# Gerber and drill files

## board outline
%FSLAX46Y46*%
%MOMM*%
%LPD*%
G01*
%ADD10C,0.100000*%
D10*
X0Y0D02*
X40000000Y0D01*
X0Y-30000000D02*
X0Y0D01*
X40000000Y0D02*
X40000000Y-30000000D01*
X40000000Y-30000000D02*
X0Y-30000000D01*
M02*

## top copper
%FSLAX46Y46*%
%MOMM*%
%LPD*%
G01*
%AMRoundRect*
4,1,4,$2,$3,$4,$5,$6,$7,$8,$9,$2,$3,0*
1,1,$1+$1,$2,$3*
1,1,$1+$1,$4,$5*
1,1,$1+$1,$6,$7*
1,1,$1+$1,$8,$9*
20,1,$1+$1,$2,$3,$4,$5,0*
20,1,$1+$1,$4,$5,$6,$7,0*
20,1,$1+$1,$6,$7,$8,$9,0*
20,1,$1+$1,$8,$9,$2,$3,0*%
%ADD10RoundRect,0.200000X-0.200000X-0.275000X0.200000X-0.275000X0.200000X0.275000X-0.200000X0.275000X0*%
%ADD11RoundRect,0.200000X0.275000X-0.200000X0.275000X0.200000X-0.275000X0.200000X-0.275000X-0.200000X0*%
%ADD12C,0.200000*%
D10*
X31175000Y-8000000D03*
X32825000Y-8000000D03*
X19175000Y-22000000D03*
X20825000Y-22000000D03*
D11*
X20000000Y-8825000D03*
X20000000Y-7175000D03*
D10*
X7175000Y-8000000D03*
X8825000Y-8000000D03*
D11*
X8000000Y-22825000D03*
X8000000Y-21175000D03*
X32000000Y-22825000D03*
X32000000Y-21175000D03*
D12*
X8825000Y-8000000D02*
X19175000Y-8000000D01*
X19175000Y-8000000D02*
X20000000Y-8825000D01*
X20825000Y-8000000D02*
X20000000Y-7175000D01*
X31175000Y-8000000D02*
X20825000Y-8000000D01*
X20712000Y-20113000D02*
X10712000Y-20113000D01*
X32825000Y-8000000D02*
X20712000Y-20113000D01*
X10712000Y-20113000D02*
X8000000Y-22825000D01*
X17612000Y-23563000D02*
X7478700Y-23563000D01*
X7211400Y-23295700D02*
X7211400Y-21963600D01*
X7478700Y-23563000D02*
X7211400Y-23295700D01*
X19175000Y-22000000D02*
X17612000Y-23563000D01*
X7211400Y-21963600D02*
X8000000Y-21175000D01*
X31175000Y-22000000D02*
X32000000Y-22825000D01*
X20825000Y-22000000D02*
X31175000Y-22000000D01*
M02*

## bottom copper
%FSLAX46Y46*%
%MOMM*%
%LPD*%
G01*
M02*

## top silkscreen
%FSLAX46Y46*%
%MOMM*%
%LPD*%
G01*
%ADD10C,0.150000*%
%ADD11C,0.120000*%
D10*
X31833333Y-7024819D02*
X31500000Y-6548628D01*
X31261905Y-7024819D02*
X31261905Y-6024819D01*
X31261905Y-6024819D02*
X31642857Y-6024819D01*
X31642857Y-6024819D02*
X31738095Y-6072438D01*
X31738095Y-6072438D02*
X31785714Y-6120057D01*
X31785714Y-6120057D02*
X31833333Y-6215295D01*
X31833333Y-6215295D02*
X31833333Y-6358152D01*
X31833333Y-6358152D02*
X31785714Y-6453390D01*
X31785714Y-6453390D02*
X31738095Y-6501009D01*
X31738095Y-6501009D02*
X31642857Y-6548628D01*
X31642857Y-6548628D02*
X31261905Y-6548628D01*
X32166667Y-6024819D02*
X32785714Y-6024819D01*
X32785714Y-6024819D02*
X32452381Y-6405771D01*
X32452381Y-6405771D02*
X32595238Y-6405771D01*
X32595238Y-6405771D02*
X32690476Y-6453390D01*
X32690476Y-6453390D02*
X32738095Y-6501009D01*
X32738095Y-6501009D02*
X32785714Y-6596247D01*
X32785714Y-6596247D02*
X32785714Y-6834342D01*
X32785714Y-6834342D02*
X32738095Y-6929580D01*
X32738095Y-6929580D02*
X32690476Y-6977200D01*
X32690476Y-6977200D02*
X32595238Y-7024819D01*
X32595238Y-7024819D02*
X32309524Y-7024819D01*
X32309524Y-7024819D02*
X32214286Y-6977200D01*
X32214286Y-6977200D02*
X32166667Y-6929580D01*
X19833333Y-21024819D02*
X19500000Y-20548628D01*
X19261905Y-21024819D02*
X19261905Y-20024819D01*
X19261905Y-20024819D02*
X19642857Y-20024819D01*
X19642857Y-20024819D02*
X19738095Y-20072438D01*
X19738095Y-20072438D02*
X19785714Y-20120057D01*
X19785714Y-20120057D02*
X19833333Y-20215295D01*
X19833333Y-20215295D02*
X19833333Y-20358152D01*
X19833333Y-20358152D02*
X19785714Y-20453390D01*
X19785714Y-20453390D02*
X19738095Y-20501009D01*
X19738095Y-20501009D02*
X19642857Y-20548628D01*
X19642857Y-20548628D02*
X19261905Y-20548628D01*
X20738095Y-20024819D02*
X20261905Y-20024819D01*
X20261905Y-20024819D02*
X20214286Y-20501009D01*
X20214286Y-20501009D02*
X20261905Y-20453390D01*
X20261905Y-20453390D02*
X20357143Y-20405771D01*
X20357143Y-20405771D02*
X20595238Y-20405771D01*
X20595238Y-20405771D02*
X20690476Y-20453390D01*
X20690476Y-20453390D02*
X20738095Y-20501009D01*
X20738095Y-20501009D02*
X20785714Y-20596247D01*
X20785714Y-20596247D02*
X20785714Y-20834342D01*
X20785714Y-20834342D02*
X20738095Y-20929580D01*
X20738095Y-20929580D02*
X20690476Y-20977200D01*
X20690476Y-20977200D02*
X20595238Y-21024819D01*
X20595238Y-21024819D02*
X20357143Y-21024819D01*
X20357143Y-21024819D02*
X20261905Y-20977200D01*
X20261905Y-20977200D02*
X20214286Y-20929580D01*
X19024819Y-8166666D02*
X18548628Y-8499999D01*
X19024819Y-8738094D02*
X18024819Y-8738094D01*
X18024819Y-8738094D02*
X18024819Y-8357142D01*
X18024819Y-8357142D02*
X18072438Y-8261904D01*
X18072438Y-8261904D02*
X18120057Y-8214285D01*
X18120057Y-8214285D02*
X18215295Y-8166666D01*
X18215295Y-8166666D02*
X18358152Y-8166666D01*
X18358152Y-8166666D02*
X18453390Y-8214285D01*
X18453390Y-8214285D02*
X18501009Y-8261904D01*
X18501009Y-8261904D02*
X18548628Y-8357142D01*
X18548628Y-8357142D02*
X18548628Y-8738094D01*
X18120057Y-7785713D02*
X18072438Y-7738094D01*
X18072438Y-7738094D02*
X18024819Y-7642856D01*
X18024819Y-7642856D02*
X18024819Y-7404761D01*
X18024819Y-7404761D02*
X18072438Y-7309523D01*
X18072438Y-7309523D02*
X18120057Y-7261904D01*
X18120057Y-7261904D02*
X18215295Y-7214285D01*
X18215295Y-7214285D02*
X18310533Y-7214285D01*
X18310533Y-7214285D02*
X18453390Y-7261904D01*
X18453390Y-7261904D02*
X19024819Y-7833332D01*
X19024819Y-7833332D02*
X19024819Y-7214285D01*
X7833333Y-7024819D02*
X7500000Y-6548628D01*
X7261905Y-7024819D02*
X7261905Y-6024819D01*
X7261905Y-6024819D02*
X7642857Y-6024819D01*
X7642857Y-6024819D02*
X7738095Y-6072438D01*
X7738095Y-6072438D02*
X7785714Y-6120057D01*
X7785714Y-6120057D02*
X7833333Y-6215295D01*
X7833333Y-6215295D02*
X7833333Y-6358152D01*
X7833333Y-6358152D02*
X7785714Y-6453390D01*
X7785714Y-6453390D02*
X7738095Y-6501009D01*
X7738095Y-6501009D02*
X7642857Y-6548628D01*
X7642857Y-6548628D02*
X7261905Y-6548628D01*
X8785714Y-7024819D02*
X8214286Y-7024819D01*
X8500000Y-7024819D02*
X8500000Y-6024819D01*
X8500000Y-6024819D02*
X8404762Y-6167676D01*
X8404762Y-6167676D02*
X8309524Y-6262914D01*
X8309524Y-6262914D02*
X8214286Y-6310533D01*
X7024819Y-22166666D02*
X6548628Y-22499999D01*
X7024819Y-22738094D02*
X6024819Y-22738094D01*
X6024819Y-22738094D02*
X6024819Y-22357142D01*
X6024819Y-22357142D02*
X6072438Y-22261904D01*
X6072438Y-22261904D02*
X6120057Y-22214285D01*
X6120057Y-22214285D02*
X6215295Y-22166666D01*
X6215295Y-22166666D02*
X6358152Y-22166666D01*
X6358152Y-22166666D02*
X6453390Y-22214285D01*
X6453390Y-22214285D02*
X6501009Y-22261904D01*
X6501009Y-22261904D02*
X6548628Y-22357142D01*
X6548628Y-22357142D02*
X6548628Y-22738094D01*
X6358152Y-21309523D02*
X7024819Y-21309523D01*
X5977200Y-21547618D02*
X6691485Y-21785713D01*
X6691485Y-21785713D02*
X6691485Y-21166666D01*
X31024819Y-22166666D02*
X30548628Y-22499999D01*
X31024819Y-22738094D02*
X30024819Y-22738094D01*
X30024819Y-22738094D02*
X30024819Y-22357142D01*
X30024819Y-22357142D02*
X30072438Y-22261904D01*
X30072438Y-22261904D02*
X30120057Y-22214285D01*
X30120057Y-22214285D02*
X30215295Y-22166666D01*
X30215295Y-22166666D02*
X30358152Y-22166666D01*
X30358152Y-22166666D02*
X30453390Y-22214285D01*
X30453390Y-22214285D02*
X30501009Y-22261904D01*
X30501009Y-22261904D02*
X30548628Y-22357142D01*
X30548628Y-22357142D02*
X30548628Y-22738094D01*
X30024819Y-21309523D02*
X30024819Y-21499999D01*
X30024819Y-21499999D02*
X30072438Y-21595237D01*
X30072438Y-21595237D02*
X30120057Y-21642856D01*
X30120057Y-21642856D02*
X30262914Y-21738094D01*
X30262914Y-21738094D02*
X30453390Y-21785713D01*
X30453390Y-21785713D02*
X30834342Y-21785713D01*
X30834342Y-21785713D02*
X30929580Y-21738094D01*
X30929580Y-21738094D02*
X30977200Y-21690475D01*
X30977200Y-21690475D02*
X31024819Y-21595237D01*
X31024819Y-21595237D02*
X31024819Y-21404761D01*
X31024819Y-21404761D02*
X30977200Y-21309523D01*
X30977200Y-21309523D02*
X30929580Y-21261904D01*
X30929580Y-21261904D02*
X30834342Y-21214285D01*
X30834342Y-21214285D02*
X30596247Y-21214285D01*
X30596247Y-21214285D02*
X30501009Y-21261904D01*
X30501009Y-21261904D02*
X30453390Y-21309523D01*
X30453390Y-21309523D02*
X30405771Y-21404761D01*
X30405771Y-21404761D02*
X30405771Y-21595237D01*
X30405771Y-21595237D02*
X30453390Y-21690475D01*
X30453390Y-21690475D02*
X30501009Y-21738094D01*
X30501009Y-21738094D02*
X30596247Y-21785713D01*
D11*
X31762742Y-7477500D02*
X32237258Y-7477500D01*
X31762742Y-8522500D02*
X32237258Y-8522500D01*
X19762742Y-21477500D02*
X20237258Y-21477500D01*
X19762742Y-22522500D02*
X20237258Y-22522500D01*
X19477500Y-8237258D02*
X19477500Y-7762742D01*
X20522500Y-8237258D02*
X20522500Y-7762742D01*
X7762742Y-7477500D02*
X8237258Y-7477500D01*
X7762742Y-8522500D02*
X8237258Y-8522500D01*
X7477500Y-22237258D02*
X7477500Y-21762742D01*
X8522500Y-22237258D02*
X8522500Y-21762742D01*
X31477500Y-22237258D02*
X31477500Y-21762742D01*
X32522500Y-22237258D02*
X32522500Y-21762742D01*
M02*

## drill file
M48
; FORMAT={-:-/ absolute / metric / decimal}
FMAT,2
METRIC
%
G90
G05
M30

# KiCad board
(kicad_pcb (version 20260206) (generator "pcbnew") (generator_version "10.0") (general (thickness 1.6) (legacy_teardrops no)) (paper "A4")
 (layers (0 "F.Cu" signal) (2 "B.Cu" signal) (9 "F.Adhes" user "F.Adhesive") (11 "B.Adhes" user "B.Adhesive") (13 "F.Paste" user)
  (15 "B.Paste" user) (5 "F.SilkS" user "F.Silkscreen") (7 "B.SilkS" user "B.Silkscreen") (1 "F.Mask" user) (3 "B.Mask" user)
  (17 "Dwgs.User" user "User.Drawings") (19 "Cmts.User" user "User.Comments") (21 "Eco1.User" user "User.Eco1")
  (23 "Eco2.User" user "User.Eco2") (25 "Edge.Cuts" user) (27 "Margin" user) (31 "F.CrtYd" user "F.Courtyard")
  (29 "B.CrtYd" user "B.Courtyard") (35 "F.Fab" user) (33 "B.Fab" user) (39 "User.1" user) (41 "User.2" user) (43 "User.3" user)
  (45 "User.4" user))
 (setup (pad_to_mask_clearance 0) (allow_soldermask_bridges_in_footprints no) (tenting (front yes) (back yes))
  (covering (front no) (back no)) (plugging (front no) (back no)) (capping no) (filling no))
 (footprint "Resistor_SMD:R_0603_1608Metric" (layer "F.Cu") (at 32 8)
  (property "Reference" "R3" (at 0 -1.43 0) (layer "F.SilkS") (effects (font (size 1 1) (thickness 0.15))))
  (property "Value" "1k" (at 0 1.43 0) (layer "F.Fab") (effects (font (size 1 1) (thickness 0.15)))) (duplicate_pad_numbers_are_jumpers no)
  (fp_line (start -0.237258 -0.5225) (end 0.237258 -0.5225) (stroke (width 0.12) (type solid)) (layer "F.SilkS"))
  (fp_line (start -0.237258 0.5225) (end 0.237258 0.5225) (stroke (width 0.12) (type solid)) (layer "F.SilkS"))
  (pad "1" smd roundrect (at -0.825 0) (size 0.8 0.95) (layers "F.Cu" "F.Mask" "F.Paste") (roundrect_rratio 0.25) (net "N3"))
  (pad "2" smd roundrect (at 0.825 0) (size 0.8 0.95) (layers "F.Cu" "F.Mask" "F.Paste") (roundrect_rratio 0.25) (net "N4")))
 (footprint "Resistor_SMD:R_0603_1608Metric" (layer "F.Cu") (at 20 22)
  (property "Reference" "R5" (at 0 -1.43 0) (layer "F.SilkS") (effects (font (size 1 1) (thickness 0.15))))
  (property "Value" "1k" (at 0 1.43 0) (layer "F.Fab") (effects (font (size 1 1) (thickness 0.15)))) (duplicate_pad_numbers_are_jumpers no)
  (fp_line (start -0.237258 -0.5225) (end 0.237258 -0.5225) (stroke (width 0.12) (type solid)) (layer "F.SilkS"))
  (fp_line (start -0.237258 0.5225) (end 0.237258 0.5225) (stroke (width 0.12) (type solid)) (layer "F.SilkS"))
  (pad "1" smd roundrect (at -0.825 0) (size 0.8 0.95) (layers "F.Cu" "F.Mask" "F.Paste") (roundrect_rratio 0.25) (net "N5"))
  (pad "2" smd roundrect (at 0.825 0) (size 0.8 0.95) (layers "F.Cu" "F.Mask" "F.Paste") (roundrect_rratio 0.25) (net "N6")))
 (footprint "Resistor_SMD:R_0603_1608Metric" (layer "F.Cu") (at 20 8 90)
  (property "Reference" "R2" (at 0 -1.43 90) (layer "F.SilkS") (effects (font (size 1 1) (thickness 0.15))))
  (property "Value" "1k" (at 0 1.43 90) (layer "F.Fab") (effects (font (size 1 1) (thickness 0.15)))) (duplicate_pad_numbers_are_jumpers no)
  (fp_line (start -0.237258 -0.5225) (end 0.237258 -0.5225) (stroke (width 0.12) (type solid)) (layer "F.SilkS"))
  (fp_line (start -0.237258 0.5225) (end 0.237258 0.5225) (stroke (width 0.12) (type solid)) (layer "F.SilkS"))
  (pad "1" smd roundrect (at -0.825 0 90) (size 0.8 0.95) (layers "F.Cu" "F.Mask" "F.Paste") (roundrect_rratio 0.25) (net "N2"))
  (pad "2" smd roundrect (at 0.825 0 90) (size 0.8 0.95) (layers "F.Cu" "F.Mask" "F.Paste") (roundrect_rratio 0.25) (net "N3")))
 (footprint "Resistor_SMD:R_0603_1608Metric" (layer "F.Cu") (at 8 8)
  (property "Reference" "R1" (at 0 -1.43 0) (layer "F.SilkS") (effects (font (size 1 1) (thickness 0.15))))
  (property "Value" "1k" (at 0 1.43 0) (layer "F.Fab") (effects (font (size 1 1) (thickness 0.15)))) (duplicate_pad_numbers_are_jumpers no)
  (fp_line (start -0.237258 -0.5225) (end 0.237258 -0.5225) (stroke (width 0.12) (type solid)) (layer "F.SilkS"))
  (fp_line (start -0.237258 0.5225) (end 0.237258 0.5225) (stroke (width 0.12) (type solid)) (layer "F.SilkS"))
  (pad "1" smd roundrect (at -0.825 0) (size 0.8 0.95) (layers "F.Cu" "F.Mask" "F.Paste") (roundrect_rratio 0.25) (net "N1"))
  (pad "2" smd roundrect (at 0.825 0) (size 0.8 0.95) (layers "F.Cu" "F.Mask" "F.Paste") (roundrect_rratio 0.25) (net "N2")))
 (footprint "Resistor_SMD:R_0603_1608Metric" (layer "F.Cu") (at 8 22 90)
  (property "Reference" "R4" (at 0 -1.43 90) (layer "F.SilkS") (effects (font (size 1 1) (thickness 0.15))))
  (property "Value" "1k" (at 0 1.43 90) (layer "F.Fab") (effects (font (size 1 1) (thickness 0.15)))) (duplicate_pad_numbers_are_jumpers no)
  (fp_line (start -0.237258 -0.5225) (end 0.237258 -0.5225) (stroke (width 0.12) (type solid)) (layer "F.SilkS"))
  (fp_line (start -0.237258 0.5225) (end 0.237258 0.5225) (stroke (width 0.12) (type solid)) (layer "F.SilkS"))
  (pad "1" smd roundrect (at -0.825 0 90) (size 0.8 0.95) (layers "F.Cu" "F.Mask" "F.Paste") (roundrect_rratio 0.25) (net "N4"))
  (pad "2" smd roundrect (at 0.825 0 90) (size 0.8 0.95) (layers "F.Cu" "F.Mask" "F.Paste") (roundrect_rratio 0.25) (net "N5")))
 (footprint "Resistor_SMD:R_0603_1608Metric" (layer "F.Cu") (at 32 22 90)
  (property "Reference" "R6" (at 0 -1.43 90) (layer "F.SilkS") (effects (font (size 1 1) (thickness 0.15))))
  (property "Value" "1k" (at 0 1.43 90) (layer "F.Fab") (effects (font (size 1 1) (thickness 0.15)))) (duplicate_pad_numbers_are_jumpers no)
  (fp_line (start -0.237258 -0.5225) (end 0.237258 -0.5225) (stroke (width 0.12) (type solid)) (layer "F.SilkS"))
  (fp_line (start -0.237258 0.5225) (end 0.237258 0.5225) (stroke (width 0.12) (type solid)) (layer "F.SilkS"))
  (pad "1" smd roundrect (at -0.825 0 90) (size 0.8 0.95) (layers "F.Cu" "F.Mask" "F.Paste") (roundrect_rratio 0.25) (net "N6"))
  (pad "2" smd roundrect (at 0.825 0 90) (size 0.8 0.95) (layers "F.Cu" "F.Mask" "F.Paste") (roundrect_rratio 0.25) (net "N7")))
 (gr_line (start 0 0) (end 40 0) (stroke (width 0.1) (type default)) (layer "Edge.Cuts"))
 (gr_line (start 0 30) (end 0 0) (stroke (width 0.1) (type default)) (layer "Edge.Cuts"))
 (gr_line (start 40 0) (end 40 30) (stroke (width 0.1) (type default)) (layer "Edge.Cuts"))
 (gr_line (start 40 30) (end 0 30) (stroke (width 0.1) (type default)) (layer "Edge.Cuts"))
 (segment (start 8.825 8) (end 19.175 8) (width 0.2) (layer "F.Cu") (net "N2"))
 (segment (start 19.175 8) (end 20 8.825) (width 0.2) (layer "F.Cu") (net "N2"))
 (segment (start 20.825 8) (end 20 7.175) (width 0.2) (layer "F.Cu") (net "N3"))
 (segment (start 31.175 8) (end 20.825 8) (width 0.2) (layer "F.Cu") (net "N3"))
 (segment (start 20.712 20.113) (end 10.712 20.113) (width 0.2) (layer "F.Cu") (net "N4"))
 (segment (start 32.825 8) (end 20.712 20.113) (width 0.2) (layer "F.Cu") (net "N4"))
 (segment (start 10.712 20.113) (end 8 22.825) (width 0.2) (layer "F.Cu") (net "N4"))
 (segment (start 17.612 23.563) (end 7.4787 23.563) (width 0.2) (layer "F.Cu") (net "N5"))
 (segment (start 7.2114 23.2957) (end 7.2114 21.9636) (width 0.2) (layer "F.Cu") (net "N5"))
 (segment (start 7.4787 23.563) (end 7.2114 23.2957) (width 0.2) (layer "F.Cu") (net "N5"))
 (segment (start 19.175 22) (end 17.612 23.563) (width 0.2) (layer "F.Cu") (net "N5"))
 (segment (start 7.2114 21.9636) (end 8 21.175) (width 0.2) (layer "F.Cu") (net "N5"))
 (segment (start 31.175 22) (end 32 22.825) (width 0.2) (layer "F.Cu") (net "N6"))
 (segment (start 20.825 22) (end 31.175 22) (width 0.2) (layer "F.Cu") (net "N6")))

